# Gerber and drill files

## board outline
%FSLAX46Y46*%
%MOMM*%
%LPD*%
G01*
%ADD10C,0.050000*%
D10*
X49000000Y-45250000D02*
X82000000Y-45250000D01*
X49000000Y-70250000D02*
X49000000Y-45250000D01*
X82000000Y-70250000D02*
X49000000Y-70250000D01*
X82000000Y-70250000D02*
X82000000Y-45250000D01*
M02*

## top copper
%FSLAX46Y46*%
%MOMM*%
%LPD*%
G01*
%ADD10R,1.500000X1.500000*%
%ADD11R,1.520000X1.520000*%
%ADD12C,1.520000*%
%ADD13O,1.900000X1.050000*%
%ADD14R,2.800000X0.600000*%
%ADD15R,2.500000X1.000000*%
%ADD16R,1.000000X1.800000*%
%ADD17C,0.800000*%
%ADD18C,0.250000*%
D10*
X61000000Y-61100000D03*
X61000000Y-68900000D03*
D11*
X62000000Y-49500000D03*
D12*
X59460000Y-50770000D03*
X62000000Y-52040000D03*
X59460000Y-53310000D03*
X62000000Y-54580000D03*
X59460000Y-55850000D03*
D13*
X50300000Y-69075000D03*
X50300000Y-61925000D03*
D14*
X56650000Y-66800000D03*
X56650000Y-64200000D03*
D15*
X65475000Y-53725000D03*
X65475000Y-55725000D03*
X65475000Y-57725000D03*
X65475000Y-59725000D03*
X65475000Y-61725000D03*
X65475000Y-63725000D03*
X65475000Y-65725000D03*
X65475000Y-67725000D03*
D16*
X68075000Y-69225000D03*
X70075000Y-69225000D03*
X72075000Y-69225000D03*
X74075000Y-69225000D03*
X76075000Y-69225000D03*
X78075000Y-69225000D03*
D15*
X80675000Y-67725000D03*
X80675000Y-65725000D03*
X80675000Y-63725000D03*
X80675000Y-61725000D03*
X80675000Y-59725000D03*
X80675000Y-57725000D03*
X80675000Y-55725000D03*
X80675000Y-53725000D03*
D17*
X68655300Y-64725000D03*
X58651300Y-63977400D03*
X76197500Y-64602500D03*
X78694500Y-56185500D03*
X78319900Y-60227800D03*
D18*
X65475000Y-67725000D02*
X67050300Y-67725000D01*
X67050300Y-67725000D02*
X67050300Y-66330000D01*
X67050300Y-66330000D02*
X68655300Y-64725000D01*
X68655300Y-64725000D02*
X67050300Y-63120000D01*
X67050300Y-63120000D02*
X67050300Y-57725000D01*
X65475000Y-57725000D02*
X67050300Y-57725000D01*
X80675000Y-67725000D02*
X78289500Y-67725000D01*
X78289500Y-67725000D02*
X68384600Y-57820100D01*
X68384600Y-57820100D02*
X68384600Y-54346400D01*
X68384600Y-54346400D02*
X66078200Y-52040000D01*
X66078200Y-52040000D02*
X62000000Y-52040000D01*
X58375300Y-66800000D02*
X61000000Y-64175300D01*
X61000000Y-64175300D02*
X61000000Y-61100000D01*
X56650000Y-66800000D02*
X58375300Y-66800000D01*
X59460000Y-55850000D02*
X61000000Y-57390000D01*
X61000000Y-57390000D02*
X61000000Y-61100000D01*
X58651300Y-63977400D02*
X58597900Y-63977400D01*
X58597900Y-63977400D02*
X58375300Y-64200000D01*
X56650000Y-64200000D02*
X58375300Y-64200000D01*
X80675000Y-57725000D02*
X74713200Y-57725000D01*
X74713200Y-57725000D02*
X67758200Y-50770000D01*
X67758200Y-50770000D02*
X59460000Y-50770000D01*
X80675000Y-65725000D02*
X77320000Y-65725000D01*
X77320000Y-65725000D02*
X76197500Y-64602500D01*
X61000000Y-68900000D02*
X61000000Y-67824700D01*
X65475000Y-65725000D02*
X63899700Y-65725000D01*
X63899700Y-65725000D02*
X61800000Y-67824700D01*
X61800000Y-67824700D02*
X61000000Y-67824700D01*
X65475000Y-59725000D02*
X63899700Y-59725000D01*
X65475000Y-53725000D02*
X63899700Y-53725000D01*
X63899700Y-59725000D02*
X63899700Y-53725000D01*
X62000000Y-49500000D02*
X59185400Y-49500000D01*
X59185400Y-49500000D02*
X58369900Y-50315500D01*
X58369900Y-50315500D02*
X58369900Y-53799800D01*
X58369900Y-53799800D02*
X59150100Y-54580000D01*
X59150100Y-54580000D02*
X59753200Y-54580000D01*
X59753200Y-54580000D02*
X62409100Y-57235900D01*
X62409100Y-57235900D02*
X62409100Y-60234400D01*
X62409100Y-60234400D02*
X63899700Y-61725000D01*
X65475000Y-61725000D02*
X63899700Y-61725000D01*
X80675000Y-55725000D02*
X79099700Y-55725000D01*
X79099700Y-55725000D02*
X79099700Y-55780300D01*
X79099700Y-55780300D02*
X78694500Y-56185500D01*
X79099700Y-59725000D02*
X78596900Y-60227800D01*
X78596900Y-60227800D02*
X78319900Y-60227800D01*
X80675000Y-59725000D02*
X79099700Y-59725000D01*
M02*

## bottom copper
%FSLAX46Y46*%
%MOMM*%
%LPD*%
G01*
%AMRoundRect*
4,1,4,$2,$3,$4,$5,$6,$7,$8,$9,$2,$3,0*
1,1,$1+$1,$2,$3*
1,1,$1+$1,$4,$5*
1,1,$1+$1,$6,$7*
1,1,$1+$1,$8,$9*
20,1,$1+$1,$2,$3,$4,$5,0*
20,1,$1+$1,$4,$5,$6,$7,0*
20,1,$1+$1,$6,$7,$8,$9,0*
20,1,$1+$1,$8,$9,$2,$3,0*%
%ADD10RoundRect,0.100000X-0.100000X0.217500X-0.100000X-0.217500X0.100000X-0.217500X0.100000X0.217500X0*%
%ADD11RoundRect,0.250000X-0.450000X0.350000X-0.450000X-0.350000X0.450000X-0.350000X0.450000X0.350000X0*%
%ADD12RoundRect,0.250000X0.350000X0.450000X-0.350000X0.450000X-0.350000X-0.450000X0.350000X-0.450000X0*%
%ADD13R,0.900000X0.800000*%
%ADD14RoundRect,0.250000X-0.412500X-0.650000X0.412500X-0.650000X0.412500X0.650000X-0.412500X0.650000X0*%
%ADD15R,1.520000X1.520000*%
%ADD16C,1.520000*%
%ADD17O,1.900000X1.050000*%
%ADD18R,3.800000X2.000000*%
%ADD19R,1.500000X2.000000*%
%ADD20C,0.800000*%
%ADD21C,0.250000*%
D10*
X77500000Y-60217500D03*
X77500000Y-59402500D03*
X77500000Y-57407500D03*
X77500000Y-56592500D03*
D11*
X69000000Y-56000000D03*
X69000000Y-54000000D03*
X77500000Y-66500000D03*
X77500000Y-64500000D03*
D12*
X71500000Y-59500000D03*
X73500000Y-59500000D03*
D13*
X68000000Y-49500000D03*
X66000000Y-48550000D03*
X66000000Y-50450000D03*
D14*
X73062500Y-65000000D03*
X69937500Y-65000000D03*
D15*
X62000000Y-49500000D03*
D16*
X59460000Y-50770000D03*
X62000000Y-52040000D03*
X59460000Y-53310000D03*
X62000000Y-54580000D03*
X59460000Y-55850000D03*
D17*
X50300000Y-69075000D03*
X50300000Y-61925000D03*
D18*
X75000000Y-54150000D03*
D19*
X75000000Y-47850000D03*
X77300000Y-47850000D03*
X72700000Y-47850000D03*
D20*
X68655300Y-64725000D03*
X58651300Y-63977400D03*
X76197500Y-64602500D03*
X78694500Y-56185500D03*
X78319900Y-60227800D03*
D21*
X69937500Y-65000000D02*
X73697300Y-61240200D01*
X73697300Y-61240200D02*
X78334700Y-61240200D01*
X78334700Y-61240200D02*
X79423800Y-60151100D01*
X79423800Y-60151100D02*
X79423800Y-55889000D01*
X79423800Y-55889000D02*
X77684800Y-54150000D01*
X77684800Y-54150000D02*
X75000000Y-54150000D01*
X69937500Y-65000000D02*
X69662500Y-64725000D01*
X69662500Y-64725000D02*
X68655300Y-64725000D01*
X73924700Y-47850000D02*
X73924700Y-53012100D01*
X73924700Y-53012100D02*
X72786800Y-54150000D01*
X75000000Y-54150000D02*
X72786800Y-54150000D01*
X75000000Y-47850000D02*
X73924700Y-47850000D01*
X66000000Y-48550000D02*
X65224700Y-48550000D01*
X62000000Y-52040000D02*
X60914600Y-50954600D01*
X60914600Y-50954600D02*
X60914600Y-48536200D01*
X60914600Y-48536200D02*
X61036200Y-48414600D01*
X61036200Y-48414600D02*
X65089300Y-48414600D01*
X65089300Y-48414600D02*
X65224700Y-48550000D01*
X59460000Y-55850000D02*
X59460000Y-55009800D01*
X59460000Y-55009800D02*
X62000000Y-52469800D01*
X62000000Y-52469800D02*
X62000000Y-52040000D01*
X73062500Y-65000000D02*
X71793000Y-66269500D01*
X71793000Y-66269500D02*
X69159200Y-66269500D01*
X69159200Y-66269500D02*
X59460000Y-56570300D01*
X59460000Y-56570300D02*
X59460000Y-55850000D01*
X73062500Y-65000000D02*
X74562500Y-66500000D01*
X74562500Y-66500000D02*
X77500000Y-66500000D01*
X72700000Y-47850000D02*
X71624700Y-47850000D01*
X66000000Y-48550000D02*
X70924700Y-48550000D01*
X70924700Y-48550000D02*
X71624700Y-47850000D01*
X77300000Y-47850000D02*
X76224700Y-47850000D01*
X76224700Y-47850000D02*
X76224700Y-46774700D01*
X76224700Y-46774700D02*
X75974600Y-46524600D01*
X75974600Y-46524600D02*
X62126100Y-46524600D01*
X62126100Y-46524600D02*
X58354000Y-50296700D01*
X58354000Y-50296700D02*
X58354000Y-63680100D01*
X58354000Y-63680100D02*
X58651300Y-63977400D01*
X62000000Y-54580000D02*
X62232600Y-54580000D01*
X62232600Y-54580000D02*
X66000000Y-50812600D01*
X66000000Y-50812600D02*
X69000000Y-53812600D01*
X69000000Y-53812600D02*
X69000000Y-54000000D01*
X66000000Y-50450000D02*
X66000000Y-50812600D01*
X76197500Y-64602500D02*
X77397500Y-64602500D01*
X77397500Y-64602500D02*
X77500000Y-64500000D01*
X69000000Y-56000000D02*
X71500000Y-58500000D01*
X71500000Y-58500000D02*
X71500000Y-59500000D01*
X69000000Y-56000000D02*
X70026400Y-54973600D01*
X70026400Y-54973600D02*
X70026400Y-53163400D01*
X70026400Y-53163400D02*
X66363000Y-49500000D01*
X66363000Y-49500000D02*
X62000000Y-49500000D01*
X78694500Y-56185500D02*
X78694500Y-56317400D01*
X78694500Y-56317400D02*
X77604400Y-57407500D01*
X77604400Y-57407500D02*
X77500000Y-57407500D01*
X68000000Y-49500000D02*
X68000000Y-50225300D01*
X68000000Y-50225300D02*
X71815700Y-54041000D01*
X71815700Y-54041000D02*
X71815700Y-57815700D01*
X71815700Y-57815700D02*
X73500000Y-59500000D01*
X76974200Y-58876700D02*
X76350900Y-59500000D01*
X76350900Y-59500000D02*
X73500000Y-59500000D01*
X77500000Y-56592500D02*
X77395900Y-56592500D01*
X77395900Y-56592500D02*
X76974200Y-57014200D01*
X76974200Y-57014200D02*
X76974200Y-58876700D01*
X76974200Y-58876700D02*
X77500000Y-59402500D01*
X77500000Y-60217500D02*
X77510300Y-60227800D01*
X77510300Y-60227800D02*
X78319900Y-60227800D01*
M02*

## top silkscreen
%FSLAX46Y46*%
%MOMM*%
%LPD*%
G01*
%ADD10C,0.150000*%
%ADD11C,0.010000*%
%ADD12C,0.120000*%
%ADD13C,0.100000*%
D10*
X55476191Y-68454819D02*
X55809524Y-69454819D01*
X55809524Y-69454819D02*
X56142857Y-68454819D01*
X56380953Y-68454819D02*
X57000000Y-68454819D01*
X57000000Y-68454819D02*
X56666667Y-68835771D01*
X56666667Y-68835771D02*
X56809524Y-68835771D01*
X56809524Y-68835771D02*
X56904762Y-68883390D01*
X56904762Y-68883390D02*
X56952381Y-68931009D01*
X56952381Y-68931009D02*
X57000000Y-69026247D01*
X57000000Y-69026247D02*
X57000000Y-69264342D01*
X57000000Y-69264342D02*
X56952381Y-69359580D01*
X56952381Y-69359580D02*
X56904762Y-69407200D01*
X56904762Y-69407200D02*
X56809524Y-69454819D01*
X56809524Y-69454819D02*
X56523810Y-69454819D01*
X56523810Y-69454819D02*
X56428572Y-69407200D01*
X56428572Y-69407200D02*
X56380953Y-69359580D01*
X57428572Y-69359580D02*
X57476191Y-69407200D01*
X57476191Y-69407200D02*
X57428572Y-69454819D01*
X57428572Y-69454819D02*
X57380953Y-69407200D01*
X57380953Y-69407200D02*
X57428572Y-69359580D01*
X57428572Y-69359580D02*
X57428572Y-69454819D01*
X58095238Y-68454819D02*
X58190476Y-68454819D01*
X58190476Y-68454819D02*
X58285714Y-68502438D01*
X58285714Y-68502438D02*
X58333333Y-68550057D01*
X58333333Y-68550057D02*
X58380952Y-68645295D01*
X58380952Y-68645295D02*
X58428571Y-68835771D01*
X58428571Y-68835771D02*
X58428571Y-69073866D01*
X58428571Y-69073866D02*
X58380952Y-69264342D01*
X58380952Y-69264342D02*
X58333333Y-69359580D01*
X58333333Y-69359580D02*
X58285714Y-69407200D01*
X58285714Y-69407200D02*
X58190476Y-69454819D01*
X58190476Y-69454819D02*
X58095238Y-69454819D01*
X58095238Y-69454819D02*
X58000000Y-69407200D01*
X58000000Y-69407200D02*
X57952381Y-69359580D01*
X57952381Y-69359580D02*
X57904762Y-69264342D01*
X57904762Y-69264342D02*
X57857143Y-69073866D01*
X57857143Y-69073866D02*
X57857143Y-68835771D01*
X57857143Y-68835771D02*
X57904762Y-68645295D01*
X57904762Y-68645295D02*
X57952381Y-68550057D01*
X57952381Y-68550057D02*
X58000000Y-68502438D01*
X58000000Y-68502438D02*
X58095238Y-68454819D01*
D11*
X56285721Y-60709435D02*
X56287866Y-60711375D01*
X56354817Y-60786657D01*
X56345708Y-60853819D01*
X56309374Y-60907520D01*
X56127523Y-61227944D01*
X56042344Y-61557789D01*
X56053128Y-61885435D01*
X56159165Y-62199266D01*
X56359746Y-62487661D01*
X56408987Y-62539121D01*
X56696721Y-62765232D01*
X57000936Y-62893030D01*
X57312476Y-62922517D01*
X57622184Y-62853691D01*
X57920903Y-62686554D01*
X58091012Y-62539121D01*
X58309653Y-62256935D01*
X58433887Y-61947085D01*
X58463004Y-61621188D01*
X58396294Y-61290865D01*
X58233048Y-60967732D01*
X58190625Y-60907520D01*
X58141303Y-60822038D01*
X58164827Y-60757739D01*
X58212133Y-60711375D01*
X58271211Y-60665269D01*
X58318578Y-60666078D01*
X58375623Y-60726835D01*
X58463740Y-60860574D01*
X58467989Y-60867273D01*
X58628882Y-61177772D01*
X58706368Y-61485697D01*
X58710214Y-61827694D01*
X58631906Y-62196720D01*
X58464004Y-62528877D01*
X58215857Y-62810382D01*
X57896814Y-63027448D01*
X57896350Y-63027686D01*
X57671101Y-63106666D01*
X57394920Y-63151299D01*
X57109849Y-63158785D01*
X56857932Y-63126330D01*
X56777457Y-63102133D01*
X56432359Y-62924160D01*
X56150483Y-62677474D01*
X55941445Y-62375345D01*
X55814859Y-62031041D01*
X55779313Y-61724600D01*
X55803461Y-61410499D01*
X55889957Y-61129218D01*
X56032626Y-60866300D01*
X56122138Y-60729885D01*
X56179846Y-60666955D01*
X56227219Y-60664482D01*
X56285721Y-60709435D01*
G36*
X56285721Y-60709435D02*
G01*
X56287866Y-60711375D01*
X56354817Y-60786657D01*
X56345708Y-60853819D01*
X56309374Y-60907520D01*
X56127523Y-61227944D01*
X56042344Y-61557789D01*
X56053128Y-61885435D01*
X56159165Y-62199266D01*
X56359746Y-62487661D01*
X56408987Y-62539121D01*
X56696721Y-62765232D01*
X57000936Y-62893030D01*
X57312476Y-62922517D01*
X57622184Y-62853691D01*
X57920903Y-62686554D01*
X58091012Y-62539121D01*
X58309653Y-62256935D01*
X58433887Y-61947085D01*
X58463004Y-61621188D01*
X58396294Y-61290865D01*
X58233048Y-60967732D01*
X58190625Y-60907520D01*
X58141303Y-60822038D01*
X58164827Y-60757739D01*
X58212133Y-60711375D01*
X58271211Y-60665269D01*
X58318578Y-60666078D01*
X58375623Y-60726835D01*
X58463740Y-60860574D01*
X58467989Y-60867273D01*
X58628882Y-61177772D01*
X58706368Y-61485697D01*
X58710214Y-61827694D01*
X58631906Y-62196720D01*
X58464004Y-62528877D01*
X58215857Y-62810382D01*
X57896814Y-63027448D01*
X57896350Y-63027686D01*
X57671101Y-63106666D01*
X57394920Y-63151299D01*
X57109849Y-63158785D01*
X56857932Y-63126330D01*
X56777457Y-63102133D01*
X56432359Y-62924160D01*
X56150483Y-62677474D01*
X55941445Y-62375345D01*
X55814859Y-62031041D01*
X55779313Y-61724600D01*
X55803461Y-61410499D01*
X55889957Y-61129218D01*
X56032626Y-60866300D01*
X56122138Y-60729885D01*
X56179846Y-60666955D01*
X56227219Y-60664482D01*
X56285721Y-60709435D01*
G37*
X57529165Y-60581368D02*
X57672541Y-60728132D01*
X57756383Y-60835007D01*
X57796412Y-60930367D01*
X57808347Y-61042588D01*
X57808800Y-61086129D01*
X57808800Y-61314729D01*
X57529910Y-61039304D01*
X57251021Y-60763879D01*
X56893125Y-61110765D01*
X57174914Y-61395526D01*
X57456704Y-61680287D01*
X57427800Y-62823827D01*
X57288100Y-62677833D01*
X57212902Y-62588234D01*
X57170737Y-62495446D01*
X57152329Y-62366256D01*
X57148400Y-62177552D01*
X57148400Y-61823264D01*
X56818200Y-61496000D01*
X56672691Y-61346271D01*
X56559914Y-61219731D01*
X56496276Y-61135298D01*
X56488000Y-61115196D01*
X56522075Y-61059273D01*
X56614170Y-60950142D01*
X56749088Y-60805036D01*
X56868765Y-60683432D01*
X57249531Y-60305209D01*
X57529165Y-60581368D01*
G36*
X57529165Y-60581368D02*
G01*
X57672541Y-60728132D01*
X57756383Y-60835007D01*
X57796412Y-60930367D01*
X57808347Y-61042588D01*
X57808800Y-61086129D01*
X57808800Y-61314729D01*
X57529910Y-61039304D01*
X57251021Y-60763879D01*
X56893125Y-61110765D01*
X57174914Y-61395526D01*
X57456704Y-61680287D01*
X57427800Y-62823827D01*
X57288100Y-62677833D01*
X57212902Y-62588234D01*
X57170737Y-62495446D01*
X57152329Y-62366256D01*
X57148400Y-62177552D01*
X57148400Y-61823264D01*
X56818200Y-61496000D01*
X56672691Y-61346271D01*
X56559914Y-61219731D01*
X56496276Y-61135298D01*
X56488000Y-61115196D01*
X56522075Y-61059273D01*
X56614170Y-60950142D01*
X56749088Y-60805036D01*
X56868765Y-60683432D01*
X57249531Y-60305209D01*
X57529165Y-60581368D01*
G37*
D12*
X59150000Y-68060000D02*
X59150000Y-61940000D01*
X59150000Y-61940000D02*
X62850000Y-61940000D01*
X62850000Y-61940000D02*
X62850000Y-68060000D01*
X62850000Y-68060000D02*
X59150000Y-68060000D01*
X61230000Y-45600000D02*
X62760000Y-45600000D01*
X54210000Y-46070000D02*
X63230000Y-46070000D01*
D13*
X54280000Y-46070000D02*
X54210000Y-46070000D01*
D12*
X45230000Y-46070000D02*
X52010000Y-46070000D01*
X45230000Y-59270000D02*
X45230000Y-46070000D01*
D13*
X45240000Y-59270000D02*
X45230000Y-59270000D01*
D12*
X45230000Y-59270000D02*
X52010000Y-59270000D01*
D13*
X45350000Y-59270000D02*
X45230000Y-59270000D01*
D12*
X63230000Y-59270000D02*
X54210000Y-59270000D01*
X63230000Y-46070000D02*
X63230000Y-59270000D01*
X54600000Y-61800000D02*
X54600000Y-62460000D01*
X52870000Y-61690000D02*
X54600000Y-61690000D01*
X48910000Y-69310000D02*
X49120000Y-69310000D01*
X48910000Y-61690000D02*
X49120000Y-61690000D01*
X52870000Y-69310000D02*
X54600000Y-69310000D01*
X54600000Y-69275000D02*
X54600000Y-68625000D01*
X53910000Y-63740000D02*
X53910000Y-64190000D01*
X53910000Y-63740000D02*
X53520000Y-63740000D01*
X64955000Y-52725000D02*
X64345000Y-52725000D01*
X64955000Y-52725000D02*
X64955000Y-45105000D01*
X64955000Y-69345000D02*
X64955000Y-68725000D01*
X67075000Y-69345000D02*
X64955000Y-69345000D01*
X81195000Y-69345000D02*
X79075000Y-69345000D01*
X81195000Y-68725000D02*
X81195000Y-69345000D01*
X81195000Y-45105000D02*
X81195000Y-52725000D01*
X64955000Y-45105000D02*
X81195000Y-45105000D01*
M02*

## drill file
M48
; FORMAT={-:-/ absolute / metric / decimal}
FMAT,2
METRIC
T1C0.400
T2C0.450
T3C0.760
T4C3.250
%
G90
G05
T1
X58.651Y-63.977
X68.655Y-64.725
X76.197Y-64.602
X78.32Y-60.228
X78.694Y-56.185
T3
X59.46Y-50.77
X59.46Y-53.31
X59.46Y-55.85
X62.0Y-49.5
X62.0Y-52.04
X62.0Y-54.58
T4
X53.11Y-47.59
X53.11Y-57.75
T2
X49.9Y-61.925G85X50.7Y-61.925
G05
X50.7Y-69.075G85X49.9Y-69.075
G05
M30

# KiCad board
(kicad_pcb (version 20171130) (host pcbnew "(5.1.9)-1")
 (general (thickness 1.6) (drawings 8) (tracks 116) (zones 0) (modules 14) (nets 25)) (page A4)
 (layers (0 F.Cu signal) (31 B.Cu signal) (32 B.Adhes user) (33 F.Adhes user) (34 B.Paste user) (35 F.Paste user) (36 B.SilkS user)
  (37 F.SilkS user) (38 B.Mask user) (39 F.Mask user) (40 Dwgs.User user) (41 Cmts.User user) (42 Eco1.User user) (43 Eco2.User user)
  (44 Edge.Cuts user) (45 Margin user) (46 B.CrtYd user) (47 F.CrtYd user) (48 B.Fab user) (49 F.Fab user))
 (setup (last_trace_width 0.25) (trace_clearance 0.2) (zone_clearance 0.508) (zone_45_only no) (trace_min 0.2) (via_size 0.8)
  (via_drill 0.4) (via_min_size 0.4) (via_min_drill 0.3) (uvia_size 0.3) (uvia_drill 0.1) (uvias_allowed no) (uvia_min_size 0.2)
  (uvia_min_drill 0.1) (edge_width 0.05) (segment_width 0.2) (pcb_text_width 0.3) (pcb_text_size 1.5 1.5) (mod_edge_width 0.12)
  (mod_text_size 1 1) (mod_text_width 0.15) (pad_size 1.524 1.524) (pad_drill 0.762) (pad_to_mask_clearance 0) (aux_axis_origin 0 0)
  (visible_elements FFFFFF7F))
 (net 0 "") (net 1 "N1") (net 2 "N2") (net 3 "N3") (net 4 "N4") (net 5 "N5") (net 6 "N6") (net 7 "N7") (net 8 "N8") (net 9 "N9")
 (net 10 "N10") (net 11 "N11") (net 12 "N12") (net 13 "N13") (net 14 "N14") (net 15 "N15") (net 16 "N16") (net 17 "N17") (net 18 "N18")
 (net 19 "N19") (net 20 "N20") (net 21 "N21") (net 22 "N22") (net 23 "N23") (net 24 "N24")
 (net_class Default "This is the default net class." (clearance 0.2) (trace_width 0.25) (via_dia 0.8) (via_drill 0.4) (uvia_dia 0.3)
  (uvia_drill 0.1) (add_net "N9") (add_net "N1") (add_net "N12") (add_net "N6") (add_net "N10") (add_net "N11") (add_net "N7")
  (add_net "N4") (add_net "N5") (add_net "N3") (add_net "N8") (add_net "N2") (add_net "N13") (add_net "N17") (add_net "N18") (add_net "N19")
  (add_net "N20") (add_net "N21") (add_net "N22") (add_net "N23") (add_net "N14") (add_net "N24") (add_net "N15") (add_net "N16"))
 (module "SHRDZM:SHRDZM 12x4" (layer B.Cu) (at 63.75 62.5 270)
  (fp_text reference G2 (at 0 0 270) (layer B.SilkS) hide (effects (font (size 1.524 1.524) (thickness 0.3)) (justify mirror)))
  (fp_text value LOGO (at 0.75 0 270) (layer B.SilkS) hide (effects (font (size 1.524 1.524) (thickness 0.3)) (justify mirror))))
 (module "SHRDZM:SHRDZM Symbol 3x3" (layer F.Cu) (at 57.25 61.75)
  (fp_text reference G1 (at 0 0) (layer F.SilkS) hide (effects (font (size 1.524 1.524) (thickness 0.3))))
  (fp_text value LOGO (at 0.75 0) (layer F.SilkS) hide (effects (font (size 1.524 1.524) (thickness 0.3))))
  (fp_poly
   (pts (xy -0.964279 -1.040565) (xy -0.962134 -1.038625) (xy -0.895183 -0.963343) (xy -0.904292 -0.896181) (xy -0.940626 -0.84248)
    (xy -1.122477 -0.522056) (xy -1.207656 -0.192211) (xy -1.196872 0.135435) (xy -1.090835 0.449266) (xy -0.890254 0.737661)
    (xy -0.841013 0.789121) (xy -0.553279 1.015232) (xy -0.249064 1.14303) (xy 0.062476 1.172517) (xy 0.372184 1.103691)
    (xy 0.670903 0.936554) (xy 0.841012 0.789121) (xy 1.059653 0.506935) (xy 1.183887 0.197085) (xy 1.213004 -0.128812)
    (xy 1.146294 -0.459135) (xy 0.983048 -0.782268) (xy 0.940625 -0.84248) (xy 0.891303 -0.927962) (xy 0.914827 -0.992261)
    (xy 0.962133 -1.038625) (xy 1.021211 -1.084731) (xy 1.068578 -1.083922) (xy 1.125623 -1.023165) (xy 1.21374 -0.889426)
    (xy 1.217989 -0.882727) (xy 1.378882 -0.572228) (xy 1.456368 -0.264303) (xy 1.460214 0.077694) (xy 1.381906 0.44672)
    (xy 1.214004 0.778877) (xy 0.965857 1.060382) (xy 0.646814 1.277448) (xy 0.64635 1.277686) (xy 0.421101 1.356666) (xy 0.14492 1.401299)
    (xy -0.140151 1.408785) (xy -0.392068 1.37633) (xy -0.472543 1.352133) (xy -0.817641 1.17416) (xy -1.099517 0.927474)
    (xy -1.308555 0.625345) (xy -1.435141 0.281041) (xy -1.470687 -0.0254) (xy -1.446539 -0.339501) (xy -1.360043 -0.620782)
    (xy -1.217374 -0.8837) (xy -1.127862 -1.020115) (xy -1.070154 -1.083045) (xy -1.022781 -1.085518) (xy -0.964279 -1.040565))
   (layer F.SilkS) (width 0.01))
  (fp_poly
   (pts (xy 0.279165 -1.168632) (xy 0.422541 -1.021868) (xy 0.506383 -0.914993) (xy 0.546412 -0.819633) (xy 0.558347 -0.707412)
    (xy 0.5588 -0.663871) (xy 0.5588 -0.435271) (xy 0.27991 -0.710696) (xy 0.001021 -0.986121) (xy -0.356875 -0.639235)
    (xy -0.075086 -0.354474) (xy 0.206704 -0.069713) (xy 0.1778 1.073827) (xy 0.0381 0.927833) (xy -0.037098 0.838234)
    (xy -0.079263 0.745446) (xy -0.097671 0.616256) (xy -0.1016 0.427552) (xy -0.1016 0.073264) (xy -0.4318 -0.254) (xy -0.577309 -0.403729)
    (xy -0.690086 -0.530269) (xy -0.753724 -0.614702) (xy -0.762 -0.634804) (xy -0.727925 -0.690727) (xy -0.63583 -0.799858)
    (xy -0.500912 -0.944964) (xy -0.381235 -1.066568) (xy -0.000469 -1.444791) (xy 0.279165 -1.168632))
   (layer F.SilkS) (width 0.01)))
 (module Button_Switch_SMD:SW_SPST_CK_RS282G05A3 (layer F.Cu) (at 61 65 90)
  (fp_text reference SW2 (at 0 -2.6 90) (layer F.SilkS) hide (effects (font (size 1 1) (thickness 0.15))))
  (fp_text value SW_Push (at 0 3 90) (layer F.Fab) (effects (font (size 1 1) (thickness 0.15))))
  (fp_line (start -3.06 -1.85) (end 3.06 -1.85) (layer F.SilkS) (width 0.12))
  (fp_line (start 3.06 -1.85) (end 3.06 1.85) (layer F.SilkS) (width 0.12))
  (fp_line (start 3.06 1.85) (end -3.06 1.85) (layer F.SilkS) (width 0.12))
  (fp_line (start -3.06 1.85) (end -3.06 -1.85) (layer F.SilkS) (width 0.12))
  (pad 2 smd rect (at 3.9 0 90) (size 1.5 1.5) (layers F.Cu F.Paste F.Mask) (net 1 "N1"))
  (pad 1 smd rect (at -3.9 0 90) (size 1.5 1.5) (layers F.Cu F.Paste F.Mask) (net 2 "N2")))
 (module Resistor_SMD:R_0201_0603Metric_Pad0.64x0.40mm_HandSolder (layer B.Cu) (at 77.5 59.81 270)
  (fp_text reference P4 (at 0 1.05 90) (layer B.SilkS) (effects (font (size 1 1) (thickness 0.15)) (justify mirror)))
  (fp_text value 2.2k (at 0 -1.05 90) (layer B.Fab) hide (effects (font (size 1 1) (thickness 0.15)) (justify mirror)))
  (pad 2 smd roundrect (at 0.4075 0 270) (size 0.635 0.4) (layers B.Cu B.Mask) (roundrect_rratio 0.25) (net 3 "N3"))
  (pad 1 smd roundrect (at -0.4075 0 270) (size 0.635 0.4) (layers B.Cu B.Mask) (roundrect_rratio 0.25) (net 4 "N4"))
  (pad "" smd roundrect (at 0.4325 0 270) (size 0.458 0.36) (layers B.Paste) (roundrect_rratio 0.25))
  (pad "" smd roundrect (at -0.4325 0 270) (size 0.458 0.36) (layers B.Paste) (roundrect_rratio 0.25)))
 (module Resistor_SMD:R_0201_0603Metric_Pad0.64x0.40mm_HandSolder (layer B.Cu) (at 77.5 57 270)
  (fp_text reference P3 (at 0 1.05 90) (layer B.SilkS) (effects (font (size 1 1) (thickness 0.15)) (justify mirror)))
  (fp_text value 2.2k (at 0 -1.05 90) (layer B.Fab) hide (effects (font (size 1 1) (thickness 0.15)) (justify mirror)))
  (pad 2 smd roundrect (at 0.4075 0 270) (size 0.635 0.4) (layers B.Cu B.Mask) (roundrect_rratio 0.25) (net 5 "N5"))
  (pad 1 smd roundrect (at -0.4075 0 270) (size 0.635 0.4) (layers B.Cu B.Mask) (roundrect_rratio 0.25) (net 4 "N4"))
  (pad "" smd roundrect (at 0.4325 0 270) (size 0.458 0.36) (layers B.Paste) (roundrect_rratio 0.25))
  (pad "" smd roundrect (at -0.4325 0 270) (size 0.458 0.36) (layers B.Paste) (roundrect_rratio 0.25)))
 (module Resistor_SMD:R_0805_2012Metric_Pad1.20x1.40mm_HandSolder (layer B.Cu) (at 69 55 270)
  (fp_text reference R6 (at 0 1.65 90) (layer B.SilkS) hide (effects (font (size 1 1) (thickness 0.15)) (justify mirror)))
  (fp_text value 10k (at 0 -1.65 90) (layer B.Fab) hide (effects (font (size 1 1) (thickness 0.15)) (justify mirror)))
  (pad 2 smd roundrect (at 1 0 270) (size 1.2 1.4) (layers B.Cu B.Paste B.Mask) (roundrect_rratio 0.208333) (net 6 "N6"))
  (pad 1 smd roundrect (at -1 0 270) (size 1.2 1.4) (layers B.Cu B.Paste B.Mask) (roundrect_rratio 0.208333) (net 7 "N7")))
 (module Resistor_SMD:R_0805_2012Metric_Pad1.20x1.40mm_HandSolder (layer B.Cu) (at 77.5 65.5 270)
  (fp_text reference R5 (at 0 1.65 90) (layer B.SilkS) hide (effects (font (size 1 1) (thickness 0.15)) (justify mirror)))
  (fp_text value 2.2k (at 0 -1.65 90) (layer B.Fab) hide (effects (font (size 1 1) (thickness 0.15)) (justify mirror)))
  (pad 2 smd roundrect (at 1 0 270) (size 1.2 1.4) (layers B.Cu B.Paste B.Mask) (roundrect_rratio 0.208333) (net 1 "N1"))
  (pad 1 smd roundrect (at -1 0 270) (size 1.2 1.4) (layers B.Cu B.Paste B.Mask) (roundrect_rratio 0.208333) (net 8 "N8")))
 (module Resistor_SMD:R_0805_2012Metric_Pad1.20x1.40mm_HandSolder (layer B.Cu) (at 72.5 59.5 180)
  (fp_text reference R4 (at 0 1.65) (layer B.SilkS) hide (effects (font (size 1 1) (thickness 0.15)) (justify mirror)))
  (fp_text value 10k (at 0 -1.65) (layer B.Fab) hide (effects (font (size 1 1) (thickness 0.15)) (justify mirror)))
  (pad 2 smd roundrect (at 1 0 180) (size 1.2 1.4) (layers B.Cu B.Paste B.Mask) (roundrect_rratio 0.208333) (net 6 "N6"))
  (pad 1 smd roundrect (at -1 0 180) (size 1.2 1.4) (layers B.Cu B.Paste B.Mask) (roundrect_rratio 0.208333) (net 4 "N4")))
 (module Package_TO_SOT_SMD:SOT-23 (layer B.Cu) (at 67 49.5)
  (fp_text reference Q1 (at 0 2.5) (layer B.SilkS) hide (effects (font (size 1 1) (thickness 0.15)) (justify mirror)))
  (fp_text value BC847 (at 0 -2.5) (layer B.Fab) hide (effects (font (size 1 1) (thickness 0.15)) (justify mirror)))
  (pad 3 smd rect (at 1 0) (size 0.9 0.8) (layers B.Cu B.Paste B.Mask) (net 4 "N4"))
  (pad 2 smd rect (at -1 -0.95) (size 0.9 0.8) (layers B.Cu B.Paste B.Mask) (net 1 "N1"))
  (pad 1 smd rect (at -1 0.95) (size 0.9 0.8) (layers B.Cu B.Paste B.Mask) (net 7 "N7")))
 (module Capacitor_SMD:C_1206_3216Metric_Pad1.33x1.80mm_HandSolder (layer B.Cu) (at 71.5 65)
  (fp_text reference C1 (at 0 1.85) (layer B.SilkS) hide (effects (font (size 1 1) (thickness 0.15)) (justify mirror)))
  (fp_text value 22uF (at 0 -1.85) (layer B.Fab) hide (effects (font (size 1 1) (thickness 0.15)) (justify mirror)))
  (pad 2 smd roundrect (at 1.5625 0) (size 1.325 1.8) (layers B.Cu B.Paste B.Mask) (roundrect_rratio 0.188679) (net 1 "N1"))
  (pad 1 smd roundrect (at -1.5625 0) (size 1.325 1.8) (layers B.Cu B.Paste B.Mask) (roundrect_rratio 0.188679) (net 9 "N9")))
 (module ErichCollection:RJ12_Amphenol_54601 (layer F.Cu) (at 62 49.5 270)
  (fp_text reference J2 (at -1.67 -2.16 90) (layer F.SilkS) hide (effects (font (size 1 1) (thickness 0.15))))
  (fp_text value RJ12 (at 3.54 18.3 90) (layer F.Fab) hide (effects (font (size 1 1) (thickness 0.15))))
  (fp_line (start -3.9 0.77) (end -3.9 -0.76) (layer F.SilkS) (width 0.12))
  (fp_line (start -3.43 7.79) (end -3.43 -1.23) (layer F.SilkS) (width 0.12))
  (fp_line (start -3.43 7.72) (end -3.43 7.79) (layer F.SilkS) (width 0.1))
  (fp_line (start -3.43 16.77) (end -3.43 9.99) (layer F.SilkS) (width 0.12))
  (fp_line (start 9.77 16.77) (end -3.43 16.77) (layer F.SilkS) (width 0.12))
  (fp_line (start 9.77 16.76) (end 9.77 16.77) (layer F.SilkS) (width 0.1))
  (fp_line (start 9.77 16.77) (end 9.77 9.99) (layer F.SilkS) (width 0.12))
  (fp_line (start 9.77 16.65) (end 9.77 16.77) (layer F.SilkS) (width 0.1))
  (fp_line (start 9.77 -1.23) (end 9.77 7.79) (layer F.SilkS) (width 0.12))
  (fp_line (start -3.43 -1.23) (end 9.77 -1.23) (layer F.SilkS) (width 0.12))
  (pad 1 thru_hole rect (at 0 0 270) (size 1.52 1.52) (drill 0.76) (layers *.Cu *.Mask) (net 6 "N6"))
  (pad "" np_thru_hole circle (at -1.91 8.89 270) (size 3.25 3.25) (drill 3.25) (layers *.Cu *.Mask))
  (pad 2 thru_hole circle (at 1.27 2.54 270) (size 1.52 1.52) (drill 0.76) (layers *.Cu *.Mask) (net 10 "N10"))
  (pad 3 thru_hole circle (at 2.54 0 270) (size 1.52 1.52) (drill 0.76) (layers *.Cu *.Mask) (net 1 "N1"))
  (pad 4 thru_hole circle (at 3.81 2.54 270) (size 1.52 1.52) (drill 0.76) (layers *.Cu *.Mask) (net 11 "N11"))
  (pad 5 thru_hole circle (at 5.08 0 270) (size 1.52 1.52) (drill 0.76) (layers *.Cu *.Mask) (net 7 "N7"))
  (pad 6 thru_hole circle (at 6.35 2.54 270) (size 1.52 1.52) (drill 0.76) (layers *.Cu *.Mask) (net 1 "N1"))
  (pad "" np_thru_hole circle (at 8.25 8.89 270) (size 3.25 3.25) (drill 3.25) (layers *.Cu *.Mask)))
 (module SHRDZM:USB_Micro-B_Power (layer F.Cu) (at 51.5 65.5 270)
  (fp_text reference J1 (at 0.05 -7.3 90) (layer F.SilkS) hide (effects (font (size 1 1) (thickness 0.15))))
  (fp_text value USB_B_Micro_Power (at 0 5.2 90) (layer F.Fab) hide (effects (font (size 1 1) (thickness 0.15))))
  (fp_line (start -3.7 -3.1) (end -3.04 -3.1) (layer F.SilkS) (width 0.12))
  (fp_line (start -3.81 -1.37) (end -3.81 -3.1) (layer F.SilkS) (width 0.12))
  (fp_line (start 3.81 2.59) (end 3.81 2.38) (layer F.SilkS) (width 0.12))
  (fp_line (start -3.81 2.59) (end -3.81 2.38) (layer F.SilkS) (width 0.12))
  (fp_line (start 3.81 -1.37) (end 3.81 -3.1) (layer F.SilkS) (width 0.12))
  (fp_line (start 3.775 -3.1) (end 3.125 -3.1) (layer F.SilkS) (width 0.12))
  (fp_line (start -1.76 -2.41) (end -1.31 -2.41) (layer F.SilkS) (width 0.12))
  (fp_line (start -1.76 -2.41) (end -1.76 -2.02) (layer F.SilkS) (width 0.12))
  (pad "" thru_hole oval (at 3.575 1.2 270) (size 1.05 1.9) (drill oval 0.45 1.25) (layers *.Cu *.Mask))
  (pad "" thru_hole oval (at -3.575 1.2 90) (size 1.05 1.9) (drill oval 0.45 1.25) (layers *.Cu *.Mask))
  (pad 5 smd rect (at 1.3 -5.15 270) (size 0.6 2.8) (layers F.Cu F.Paste F.Mask) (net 1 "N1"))
  (pad 1 smd rect (at -1.3 -5.15 270) (size 0.6 2.8) (layers F.Cu F.Paste F.Mask) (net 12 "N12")))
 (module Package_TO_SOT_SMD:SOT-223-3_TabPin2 (layer B.Cu) (at 75 51 270)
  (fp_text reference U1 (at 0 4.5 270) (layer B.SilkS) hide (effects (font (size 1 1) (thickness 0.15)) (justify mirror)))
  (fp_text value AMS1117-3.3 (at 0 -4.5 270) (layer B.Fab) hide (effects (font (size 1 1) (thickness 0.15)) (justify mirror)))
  (pad 2 smd rect (at 3.15 0 270) (size 2 3.8) (layers B.Cu B.Paste B.Mask) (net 9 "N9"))
  (pad 2 smd rect (at -3.15 0 270) (size 2 1.5) (layers B.Cu B.Paste B.Mask) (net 9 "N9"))
  (pad 3 smd rect (at -3.15 -2.3 270) (size 2 1.5) (layers B.Cu B.Paste B.Mask) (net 12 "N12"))
  (pad 1 smd rect (at -3.15 2.3 270) (size 2 1.5) (layers B.Cu B.Paste B.Mask) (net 1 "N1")))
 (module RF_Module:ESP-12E (layer F.Cu) (at 73.075 57.225)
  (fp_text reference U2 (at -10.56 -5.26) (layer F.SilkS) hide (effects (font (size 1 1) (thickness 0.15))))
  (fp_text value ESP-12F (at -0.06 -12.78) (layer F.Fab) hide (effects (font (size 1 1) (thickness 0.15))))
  (fp_line (start -8.12 -4.5) (end -8.73 -4.5) (layer F.SilkS) (width 0.12))
  (fp_line (start -8.12 -4.5) (end -8.12 -12.12) (layer F.SilkS) (width 0.12))
  (fp_line (start -8.12 12.12) (end -8.12 11.5) (layer F.SilkS) (width 0.12))
  (fp_line (start -6 12.12) (end -8.12 12.12) (layer F.SilkS) (width 0.12))
  (fp_line (start 8.12 12.12) (end 6 12.12) (layer F.SilkS) (width 0.12))
  (fp_line (start 8.12 11.5) (end 8.12 12.12) (layer F.SilkS) (width 0.12))
  (fp_line (start 8.12 -12.12) (end 8.12 -4.5) (layer F.SilkS) (width 0.12))
  (fp_line (start -8.12 -12.12) (end 8.12 -12.12) (layer F.SilkS) (width 0.12))
  (pad 1 smd rect (at -7.6 -3.5) (size 2.5 1) (layers F.Cu F.Paste F.Mask) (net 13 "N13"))
  (pad 2 smd rect (at -7.6 -1.5) (size 2.5 1) (layers F.Cu F.Paste F.Mask) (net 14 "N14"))
  (pad 3 smd rect (at -7.6 0.5) (size 2.5 1) (layers F.Cu F.Paste F.Mask) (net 9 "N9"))
  (pad 4 smd rect (at -7.6 2.5) (size 2.5 1) (layers F.Cu F.Paste F.Mask) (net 13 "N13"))
  (pad 5 smd rect (at -7.6 4.5) (size 2.5 1) (layers F.Cu F.Paste F.Mask) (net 6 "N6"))
  (pad 6 smd rect (at -7.6 6.5) (size 2.5 1) (layers F.Cu F.Paste F.Mask) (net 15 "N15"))
  (pad 7 smd rect (at -7.6 8.5) (size 2.5 1) (layers F.Cu F.Paste F.Mask) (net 2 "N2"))
  (pad 8 smd rect (at -7.6 10.5) (size 2.5 1) (layers F.Cu F.Paste F.Mask) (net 9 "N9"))
  (pad 9 smd rect (at -5 12) (size 1 1.8) (layers F.Cu F.Paste F.Mask) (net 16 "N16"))
  (pad 10 smd rect (at -3 12) (size 1 1.8) (layers F.Cu F.Paste F.Mask) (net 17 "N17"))
  (pad 11 smd rect (at -1 12) (size 1 1.8) (layers F.Cu F.Paste F.Mask) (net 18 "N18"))
  (pad 12 smd rect (at 1 12) (size 1 1.8) (layers F.Cu F.Paste F.Mask) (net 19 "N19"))
  (pad 13 smd rect (at 3 12) (size 1 1.8) (layers F.Cu F.Paste F.Mask) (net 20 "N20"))
  (pad 14 smd rect (at 5 12) (size 1 1.8) (layers F.Cu F.Paste F.Mask) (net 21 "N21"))
  (pad 15 smd rect (at 7.6 10.5) (size 2.5 1) (layers F.Cu F.Paste F.Mask) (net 1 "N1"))
  (pad 16 smd rect (at 7.6 8.5) (size 2.5 1) (layers F.Cu F.Paste F.Mask) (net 8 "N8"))
  (pad 17 smd rect (at 7.6 6.5) (size 2.5 1) (layers F.Cu F.Paste F.Mask) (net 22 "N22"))
  (pad 18 smd rect (at 7.6 4.5) (size 2.5 1) (layers F.Cu F.Paste F.Mask) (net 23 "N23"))
  (pad 19 smd rect (at 7.6 2.5) (size 2.5 1) (layers F.Cu F.Paste F.Mask) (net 3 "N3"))
  (pad 20 smd rect (at 7.6 0.5) (size 2.5 1) (layers F.Cu F.Paste F.Mask) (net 10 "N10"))
  (pad 21 smd rect (at 7.6 -1.5) (size 2.5 1) (layers F.Cu F.Paste F.Mask) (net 5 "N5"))
  (pad 22 smd rect (at 7.6 -3.5) (size 2.5 1) (layers F.Cu F.Paste F.Mask) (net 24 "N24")))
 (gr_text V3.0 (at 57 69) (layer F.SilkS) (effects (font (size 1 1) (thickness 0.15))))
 (gr_line (start 49 45.25) (end 82 45.25) (layer Edge.Cuts) (width 0.05))
 (gr_line (start 49 70.25) (end 49 45.25) (layer Edge.Cuts) (width 0.05))
 (gr_line (start 82 70.25) (end 49 70.25) (layer Edge.Cuts) (width 0.05))
 (gr_line (start 82 70.25) (end 82 45.25) (layer Edge.Cuts) (width 0.05))
 (segment (start 65.475 67.725) (end 67.0503 67.725) (width 0.25) (layer F.Cu) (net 9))
 (segment (start 67.0503 67.725) (end 67.0503 66.33) (width 0.25) (layer F.Cu) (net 9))
 (segment (start 67.0503 66.33) (end 68.6553 64.725) (width 0.25) (layer F.Cu) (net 9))
 (segment (start 69.9375 65) (end 73.6973 61.2402) (width 0.25) (layer B.Cu) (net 9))
 (segment (start 73.6973 61.2402) (end 78.3347 61.2402) (width 0.25) (layer B.Cu) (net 9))
 (segment (start 78.3347 61.2402) (end 79.4238 60.1511) (width 0.25) (layer B.Cu) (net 9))
 (segment (start 79.4238 60.1511) (end 79.4238 55.889) (width 0.25) (layer B.Cu) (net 9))
 (segment (start 79.4238 55.889) (end 77.6848 54.15) (width 0.25) (layer B.Cu) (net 9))
 (segment (start 77.6848 54.15) (end 75 54.15) (width 0.25) (layer B.Cu) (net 9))
 (segment (start 68.6553 64.725) (end 67.0503 63.12) (width 0.25) (layer F.Cu) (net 9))
 (segment (start 67.0503 63.12) (end 67.0503 57.725) (width 0.25) (layer F.Cu) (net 9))
 (segment (start 65.475 57.725) (end 67.0503 57.725) (width 0.25) (layer F.Cu) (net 9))
 (segment (start 69.9375 65) (end 69.6625 64.725) (width 0.25) (layer B.Cu) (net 9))
 (segment (start 69.6625 64.725) (end 68.6553 64.725) (width 0.25) (layer B.Cu) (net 9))
 (segment (start 73.9247 47.85) (end 73.9247 53.0121) (width 0.25) (layer B.Cu) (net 9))
 (segment (start 73.9247 53.0121) (end 72.7868 54.15) (width 0.25) (layer B.Cu) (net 9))
 (segment (start 75 54.15) (end 72.7868 54.15) (width 0.25) (layer B.Cu) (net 9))
 (segment (start 75 47.85) (end 73.9247 47.85) (width 0.25) (layer B.Cu) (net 9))
 (via (at 68.6553 64.725) (size 0.8) (layers F.Cu B.Cu) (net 9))
 (segment (start 80.675 67.725) (end 78.2895 67.725) (width 0.25) (layer F.Cu) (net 1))
 (segment (start 78.2895 67.725) (end 68.3846 57.8201) (width 0.25) (layer F.Cu) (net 1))
 (segment (start 68.3846 57.8201) (end 68.3846 54.3464) (width 0.25) (layer F.Cu) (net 1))
 (segment (start 68.3846 54.3464) (end 66.0782 52.04) (width 0.25) (layer F.Cu) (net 1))
 (segment (start 66.0782 52.04) (end 62 52.04) (width 0.25) (layer F.Cu) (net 1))
 (segment (start 58.3753 66.8) (end 61 64.1753) (width 0.25) (layer F.Cu) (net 1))
 (segment (start 61 64.1753) (end 61 61.1) (width 0.25) (layer F.Cu) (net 1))
 (segment (start 66 48.55) (end 65.2247 48.55) (width 0.25) (layer B.Cu) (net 1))
 (segment (start 62 52.04) (end 60.9146 50.9546) (width 0.25) (layer B.Cu) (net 1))
 (segment (start 60.9146 50.9546) (end 60.9146 48.5362) (width 0.25) (layer B.Cu) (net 1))
 (segment (start 60.9146 48.5362) (end 61.0362 48.4146) (width 0.25) (layer B.Cu) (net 1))
 (segment (start 61.0362 48.4146) (end 65.0893 48.4146) (width 0.25) (layer B.Cu) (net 1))
 (segment (start 65.0893 48.4146) (end 65.2247 48.55) (width 0.25) (layer B.Cu) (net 1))
 (segment (start 59.46 55.85) (end 59.46 55.0098) (width 0.25) (layer B.Cu) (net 1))
 (segment (start 59.46 55.0098) (end 62 52.4698) (width 0.25) (layer B.Cu) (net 1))
 (segment (start 62 52.4698) (end 62 52.04) (width 0.25) (layer B.Cu) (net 1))
 (segment (start 73.0625 65) (end 71.793 66.2695) (width 0.25) (layer B.Cu) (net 1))
 (segment (start 71.793 66.2695) (end 69.1592 66.2695) (width 0.25) (layer B.Cu) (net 1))
 (segment (start 69.1592 66.2695) (end 59.46 56.5703) (width 0.25) (layer B.Cu) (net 1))
 (segment (start 59.46 56.5703) (end 59.46 55.85) (width 0.25) (layer B.Cu) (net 1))
 (segment (start 73.0625 65) (end 74.5625 66.5) (width 0.25) (layer B.Cu) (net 1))
 (segment (start 74.5625 66.5) (end 77.5 66.5) (width 0.25) (layer B.Cu) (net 1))
 (segment (start 72.7 47.85) (end 71.6247 47.85) (width 0.25) (layer B.Cu) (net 1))
 (segment (start 66 48.55) (end 70.9247 48.55) (width 0.25) (layer B.Cu) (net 1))
 (segment (start 70.9247 48.55) (end 71.6247 47.85) (width 0.25) (layer B.Cu) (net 1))
 (segment (start 56.65 66.8) (end 58.3753 66.8) (width 0.25) (layer F.Cu) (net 1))
 (segment (start 59.46 55.85) (end 61 57.39) (width 0.25) (layer F.Cu) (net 1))
 (segment (start 61 57.39) (end 61 61.1) (width 0.25) (layer F.Cu) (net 1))
 (segment (start 77.3 47.85) (end 76.2247 47.85) (width 0.25) (layer B.Cu) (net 12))
 (segment (start 58.6513 63.9774) (end 58.5979 63.9774) (width 0.25) (layer F.Cu) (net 12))
 (segment (start 58.5979 63.9774) (end 58.3753 64.2) (width 0.25) (layer F.Cu) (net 12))
 (segment (start 76.2247 47.85) (end 76.2247 46.7747) (width 0.25) (layer B.Cu) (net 12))
 (segment (start 76.2247 46.7747) (end 75.9746 46.5246) (width 0.25) (layer B.Cu) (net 12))
 (segment (start 75.9746 46.5246) (end 62.1261 46.5246) (width 0.25) (layer B.Cu) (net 12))
 (segment (start 62.1261 46.5246) (end 58.354 50.2967) (width 0.25) (layer B.Cu) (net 12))
 (segment (start 58.354 50.2967) (end 58.354 63.6801) (width 0.25) (layer B.Cu) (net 12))
 (segment (start 58.354 63.6801) (end 58.6513 63.9774) (width 0.25) (layer B.Cu) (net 12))
 (segment (start 56.65 64.2) (end 58.3753 64.2) (width 0.25) (layer F.Cu) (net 12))
 (via (at 58.6513 63.9774) (size 0.8) (layers F.Cu B.Cu) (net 12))
 (segment (start 62 54.58) (end 62.2326 54.58) (width 0.25) (layer B.Cu) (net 7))
 (segment (start 62.2326 54.58) (end 66 50.8126) (width 0.25) (layer B.Cu) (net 7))
 (segment (start 66 50.8126) (end 69 53.8126) (width 0.25) (layer B.Cu) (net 7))
 (segment (start 69 53.8126) (end 69 54) (width 0.25) (layer B.Cu) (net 7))
 (segment (start 66 50.45) (end 66 50.8126) (width 0.25) (layer B.Cu) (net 7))
 (segment (start 80.675 57.725) (end 74.7132 57.725) (width 0.25) (layer F.Cu) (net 10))
 (segment (start 74.7132 57.725) (end 67.7582 50.77) (width 0.25) (layer F.Cu) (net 10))
 (segment (start 67.7582 50.77) (end 59.46 50.77) (width 0.25) (layer F.Cu) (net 10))
 (segment (start 80.675 65.725) (end 77.32 65.725) (width 0.25) (layer F.Cu) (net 8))
 (segment (start 77.32 65.725) (end 76.1975 64.6025) (width 0.25) (layer F.Cu) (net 8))
 (segment (start 76.1975 64.6025) (end 77.3975 64.6025) (width 0.25) (layer B.Cu) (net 8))
 (segment (start 77.3975 64.6025) (end 77.5 64.5) (width 0.25) (layer B.Cu) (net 8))
 (via (at 76.1975 64.6025) (size 0.8) (layers F.Cu B.Cu) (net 8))
 (segment (start 61 68.9) (end 61 67.8247) (width 0.25) (layer F.Cu) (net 2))
 (segment (start 65.475 65.725) (end 63.8997 65.725) (width 0.25) (layer F.Cu) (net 2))
 (segment (start 63.8997 65.725) (end 61.8 67.8247) (width 0.25) (layer F.Cu) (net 2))
 (segment (start 61.8 67.8247) (end 61 67.8247) (width 0.25) (layer F.Cu) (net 2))
 (segment (start 65.475 59.725) (end 63.8997 59.725) (width 0.25) (layer F.Cu) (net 13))
 (segment (start 65.475 53.725) (end 63.8997 53.725) (width 0.25) (layer F.Cu) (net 13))
 (segment (start 63.8997 59.725) (end 63.8997 53.725) (width 0.25) (layer F.Cu) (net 13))
 (segment (start 62 49.5) (end 59.1854 49.5) (width 0.25) (layer F.Cu) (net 6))
 (segment (start 59.1854 49.5) (end 58.3699 50.3155) (width 0.25) (layer F.Cu) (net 6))
 (segment (start 58.3699 50.3155) (end 58.3699 53.7998) (width 0.25) (layer F.Cu) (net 6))
 (segment (start 58.3699 53.7998) (end 59.1501 54.58) (width 0.25) (layer F.Cu) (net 6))
 (segment (start 59.1501 54.58) (end 59.7532 54.58) (width 0.25) (layer F.Cu) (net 6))
 (segment (start 59.7532 54.58) (end 62.4091 57.2359) (width 0.25) (layer F.Cu) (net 6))
 (segment (start 62.4091 57.2359) (end 62.4091 60.2344) (width 0.25) (layer F.Cu) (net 6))
 (segment (start 62.4091 60.2344) (end 63.8997 61.725) (width 0.25) (layer F.Cu) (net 6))
 (segment (start 65.475 61.725) (end 63.8997 61.725) (width 0.25) (layer F.Cu) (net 6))
 (segment (start 69 56) (end 71.5 58.5) (width 0.25) (layer B.Cu) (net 6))
 (segment (start 71.5 58.5) (end 71.5 59.5) (width 0.25) (layer B.Cu) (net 6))
 (segment (start 69 56) (end 70.0264 54.9736) (width 0.25) (layer B.Cu) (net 6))
 (segment (start 70.0264 54.9736) (end 70.0264 53.1634) (width 0.25) (layer B.Cu) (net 6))
 (segment (start 70.0264 53.1634) (end 66.363 49.5) (width 0.25) (layer B.Cu) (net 6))
 (segment (start 66.363 49.5) (end 62 49.5) (width 0.25) (layer B.Cu) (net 6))
 (segment (start 80.675 55.725) (end 79.0997 55.725) (width 0.25) (layer F.Cu) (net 5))
 (segment (start 78.6945 56.1855) (end 78.6945 56.3174) (width 0.25) (layer B.Cu) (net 5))
 (segment (start 78.6945 56.3174) (end 77.6044 57.4075) (width 0.25) (layer B.Cu) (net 5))
 (segment (start 77.6044 57.4075) (end 77.5 57.4075) (width 0.25) (layer B.Cu) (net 5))
 (segment (start 79.0997 55.725) (end 79.0997 55.7803) (width 0.25) (layer F.Cu) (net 5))
 (segment (start 79.0997 55.7803) (end 78.6945 56.1855) (width 0.25) (layer F.Cu) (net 5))
 (via (at 78.6945 56.1855) (size 0.8) (layers F.Cu B.Cu) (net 5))
 (segment (start 68 49.5) (end 68 50.2253) (width 0.25) (layer B.Cu) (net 4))
 (segment (start 68 50.2253) (end 71.8157 54.041) (width 0.25) (layer B.Cu) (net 4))
 (segment (start 71.8157 54.041) (end 71.8157 57.8157) (width 0.25) (layer B.Cu) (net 4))
 (segment (start 71.8157 57.8157) (end 73.5 59.5) (width 0.25) (layer B.Cu) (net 4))
 (segment (start 76.9742 58.8767) (end 76.3509 59.5) (width 0.25) (layer B.Cu) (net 4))
 (segment (start 76.3509 59.5) (end 73.5 59.5) (width 0.25) (layer B.Cu) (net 4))
 (segment (start 77.5 56.5925) (end 77.3959 56.5925) (width 0.25) (layer B.Cu) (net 4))
 (segment (start 77.3959 56.5925) (end 76.9742 57.0142) (width 0.25) (layer B.Cu) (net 4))
 (segment (start 76.9742 57.0142) (end 76.9742 58.8767) (width 0.25) (layer B.Cu) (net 4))
 (segment (start 76.9742 58.8767) (end 77.5 59.4025) (width 0.25) (layer B.Cu) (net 4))
 (segment (start 79.0997 59.725) (end 78.5969 60.2278) (width 0.25) (layer F.Cu) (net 3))
 (segment (start 78.5969 60.2278) (end 78.3199 60.2278) (width 0.25) (layer F.Cu) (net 3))
 (segment (start 77.5 60.2175) (end 77.5103 60.2278) (width 0.25) (layer B.Cu) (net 3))
 (segment (start 77.5103 60.2278) (end 78.3199 60.2278) (width 0.25) (layer B.Cu) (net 3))
 (segment (start 80.675 59.725) (end 79.0997 59.725) (width 0.25) (layer F.Cu) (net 3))
 (via (at 78.3199 60.2278) (size 0.8) (layers F.Cu B.Cu) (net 3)))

